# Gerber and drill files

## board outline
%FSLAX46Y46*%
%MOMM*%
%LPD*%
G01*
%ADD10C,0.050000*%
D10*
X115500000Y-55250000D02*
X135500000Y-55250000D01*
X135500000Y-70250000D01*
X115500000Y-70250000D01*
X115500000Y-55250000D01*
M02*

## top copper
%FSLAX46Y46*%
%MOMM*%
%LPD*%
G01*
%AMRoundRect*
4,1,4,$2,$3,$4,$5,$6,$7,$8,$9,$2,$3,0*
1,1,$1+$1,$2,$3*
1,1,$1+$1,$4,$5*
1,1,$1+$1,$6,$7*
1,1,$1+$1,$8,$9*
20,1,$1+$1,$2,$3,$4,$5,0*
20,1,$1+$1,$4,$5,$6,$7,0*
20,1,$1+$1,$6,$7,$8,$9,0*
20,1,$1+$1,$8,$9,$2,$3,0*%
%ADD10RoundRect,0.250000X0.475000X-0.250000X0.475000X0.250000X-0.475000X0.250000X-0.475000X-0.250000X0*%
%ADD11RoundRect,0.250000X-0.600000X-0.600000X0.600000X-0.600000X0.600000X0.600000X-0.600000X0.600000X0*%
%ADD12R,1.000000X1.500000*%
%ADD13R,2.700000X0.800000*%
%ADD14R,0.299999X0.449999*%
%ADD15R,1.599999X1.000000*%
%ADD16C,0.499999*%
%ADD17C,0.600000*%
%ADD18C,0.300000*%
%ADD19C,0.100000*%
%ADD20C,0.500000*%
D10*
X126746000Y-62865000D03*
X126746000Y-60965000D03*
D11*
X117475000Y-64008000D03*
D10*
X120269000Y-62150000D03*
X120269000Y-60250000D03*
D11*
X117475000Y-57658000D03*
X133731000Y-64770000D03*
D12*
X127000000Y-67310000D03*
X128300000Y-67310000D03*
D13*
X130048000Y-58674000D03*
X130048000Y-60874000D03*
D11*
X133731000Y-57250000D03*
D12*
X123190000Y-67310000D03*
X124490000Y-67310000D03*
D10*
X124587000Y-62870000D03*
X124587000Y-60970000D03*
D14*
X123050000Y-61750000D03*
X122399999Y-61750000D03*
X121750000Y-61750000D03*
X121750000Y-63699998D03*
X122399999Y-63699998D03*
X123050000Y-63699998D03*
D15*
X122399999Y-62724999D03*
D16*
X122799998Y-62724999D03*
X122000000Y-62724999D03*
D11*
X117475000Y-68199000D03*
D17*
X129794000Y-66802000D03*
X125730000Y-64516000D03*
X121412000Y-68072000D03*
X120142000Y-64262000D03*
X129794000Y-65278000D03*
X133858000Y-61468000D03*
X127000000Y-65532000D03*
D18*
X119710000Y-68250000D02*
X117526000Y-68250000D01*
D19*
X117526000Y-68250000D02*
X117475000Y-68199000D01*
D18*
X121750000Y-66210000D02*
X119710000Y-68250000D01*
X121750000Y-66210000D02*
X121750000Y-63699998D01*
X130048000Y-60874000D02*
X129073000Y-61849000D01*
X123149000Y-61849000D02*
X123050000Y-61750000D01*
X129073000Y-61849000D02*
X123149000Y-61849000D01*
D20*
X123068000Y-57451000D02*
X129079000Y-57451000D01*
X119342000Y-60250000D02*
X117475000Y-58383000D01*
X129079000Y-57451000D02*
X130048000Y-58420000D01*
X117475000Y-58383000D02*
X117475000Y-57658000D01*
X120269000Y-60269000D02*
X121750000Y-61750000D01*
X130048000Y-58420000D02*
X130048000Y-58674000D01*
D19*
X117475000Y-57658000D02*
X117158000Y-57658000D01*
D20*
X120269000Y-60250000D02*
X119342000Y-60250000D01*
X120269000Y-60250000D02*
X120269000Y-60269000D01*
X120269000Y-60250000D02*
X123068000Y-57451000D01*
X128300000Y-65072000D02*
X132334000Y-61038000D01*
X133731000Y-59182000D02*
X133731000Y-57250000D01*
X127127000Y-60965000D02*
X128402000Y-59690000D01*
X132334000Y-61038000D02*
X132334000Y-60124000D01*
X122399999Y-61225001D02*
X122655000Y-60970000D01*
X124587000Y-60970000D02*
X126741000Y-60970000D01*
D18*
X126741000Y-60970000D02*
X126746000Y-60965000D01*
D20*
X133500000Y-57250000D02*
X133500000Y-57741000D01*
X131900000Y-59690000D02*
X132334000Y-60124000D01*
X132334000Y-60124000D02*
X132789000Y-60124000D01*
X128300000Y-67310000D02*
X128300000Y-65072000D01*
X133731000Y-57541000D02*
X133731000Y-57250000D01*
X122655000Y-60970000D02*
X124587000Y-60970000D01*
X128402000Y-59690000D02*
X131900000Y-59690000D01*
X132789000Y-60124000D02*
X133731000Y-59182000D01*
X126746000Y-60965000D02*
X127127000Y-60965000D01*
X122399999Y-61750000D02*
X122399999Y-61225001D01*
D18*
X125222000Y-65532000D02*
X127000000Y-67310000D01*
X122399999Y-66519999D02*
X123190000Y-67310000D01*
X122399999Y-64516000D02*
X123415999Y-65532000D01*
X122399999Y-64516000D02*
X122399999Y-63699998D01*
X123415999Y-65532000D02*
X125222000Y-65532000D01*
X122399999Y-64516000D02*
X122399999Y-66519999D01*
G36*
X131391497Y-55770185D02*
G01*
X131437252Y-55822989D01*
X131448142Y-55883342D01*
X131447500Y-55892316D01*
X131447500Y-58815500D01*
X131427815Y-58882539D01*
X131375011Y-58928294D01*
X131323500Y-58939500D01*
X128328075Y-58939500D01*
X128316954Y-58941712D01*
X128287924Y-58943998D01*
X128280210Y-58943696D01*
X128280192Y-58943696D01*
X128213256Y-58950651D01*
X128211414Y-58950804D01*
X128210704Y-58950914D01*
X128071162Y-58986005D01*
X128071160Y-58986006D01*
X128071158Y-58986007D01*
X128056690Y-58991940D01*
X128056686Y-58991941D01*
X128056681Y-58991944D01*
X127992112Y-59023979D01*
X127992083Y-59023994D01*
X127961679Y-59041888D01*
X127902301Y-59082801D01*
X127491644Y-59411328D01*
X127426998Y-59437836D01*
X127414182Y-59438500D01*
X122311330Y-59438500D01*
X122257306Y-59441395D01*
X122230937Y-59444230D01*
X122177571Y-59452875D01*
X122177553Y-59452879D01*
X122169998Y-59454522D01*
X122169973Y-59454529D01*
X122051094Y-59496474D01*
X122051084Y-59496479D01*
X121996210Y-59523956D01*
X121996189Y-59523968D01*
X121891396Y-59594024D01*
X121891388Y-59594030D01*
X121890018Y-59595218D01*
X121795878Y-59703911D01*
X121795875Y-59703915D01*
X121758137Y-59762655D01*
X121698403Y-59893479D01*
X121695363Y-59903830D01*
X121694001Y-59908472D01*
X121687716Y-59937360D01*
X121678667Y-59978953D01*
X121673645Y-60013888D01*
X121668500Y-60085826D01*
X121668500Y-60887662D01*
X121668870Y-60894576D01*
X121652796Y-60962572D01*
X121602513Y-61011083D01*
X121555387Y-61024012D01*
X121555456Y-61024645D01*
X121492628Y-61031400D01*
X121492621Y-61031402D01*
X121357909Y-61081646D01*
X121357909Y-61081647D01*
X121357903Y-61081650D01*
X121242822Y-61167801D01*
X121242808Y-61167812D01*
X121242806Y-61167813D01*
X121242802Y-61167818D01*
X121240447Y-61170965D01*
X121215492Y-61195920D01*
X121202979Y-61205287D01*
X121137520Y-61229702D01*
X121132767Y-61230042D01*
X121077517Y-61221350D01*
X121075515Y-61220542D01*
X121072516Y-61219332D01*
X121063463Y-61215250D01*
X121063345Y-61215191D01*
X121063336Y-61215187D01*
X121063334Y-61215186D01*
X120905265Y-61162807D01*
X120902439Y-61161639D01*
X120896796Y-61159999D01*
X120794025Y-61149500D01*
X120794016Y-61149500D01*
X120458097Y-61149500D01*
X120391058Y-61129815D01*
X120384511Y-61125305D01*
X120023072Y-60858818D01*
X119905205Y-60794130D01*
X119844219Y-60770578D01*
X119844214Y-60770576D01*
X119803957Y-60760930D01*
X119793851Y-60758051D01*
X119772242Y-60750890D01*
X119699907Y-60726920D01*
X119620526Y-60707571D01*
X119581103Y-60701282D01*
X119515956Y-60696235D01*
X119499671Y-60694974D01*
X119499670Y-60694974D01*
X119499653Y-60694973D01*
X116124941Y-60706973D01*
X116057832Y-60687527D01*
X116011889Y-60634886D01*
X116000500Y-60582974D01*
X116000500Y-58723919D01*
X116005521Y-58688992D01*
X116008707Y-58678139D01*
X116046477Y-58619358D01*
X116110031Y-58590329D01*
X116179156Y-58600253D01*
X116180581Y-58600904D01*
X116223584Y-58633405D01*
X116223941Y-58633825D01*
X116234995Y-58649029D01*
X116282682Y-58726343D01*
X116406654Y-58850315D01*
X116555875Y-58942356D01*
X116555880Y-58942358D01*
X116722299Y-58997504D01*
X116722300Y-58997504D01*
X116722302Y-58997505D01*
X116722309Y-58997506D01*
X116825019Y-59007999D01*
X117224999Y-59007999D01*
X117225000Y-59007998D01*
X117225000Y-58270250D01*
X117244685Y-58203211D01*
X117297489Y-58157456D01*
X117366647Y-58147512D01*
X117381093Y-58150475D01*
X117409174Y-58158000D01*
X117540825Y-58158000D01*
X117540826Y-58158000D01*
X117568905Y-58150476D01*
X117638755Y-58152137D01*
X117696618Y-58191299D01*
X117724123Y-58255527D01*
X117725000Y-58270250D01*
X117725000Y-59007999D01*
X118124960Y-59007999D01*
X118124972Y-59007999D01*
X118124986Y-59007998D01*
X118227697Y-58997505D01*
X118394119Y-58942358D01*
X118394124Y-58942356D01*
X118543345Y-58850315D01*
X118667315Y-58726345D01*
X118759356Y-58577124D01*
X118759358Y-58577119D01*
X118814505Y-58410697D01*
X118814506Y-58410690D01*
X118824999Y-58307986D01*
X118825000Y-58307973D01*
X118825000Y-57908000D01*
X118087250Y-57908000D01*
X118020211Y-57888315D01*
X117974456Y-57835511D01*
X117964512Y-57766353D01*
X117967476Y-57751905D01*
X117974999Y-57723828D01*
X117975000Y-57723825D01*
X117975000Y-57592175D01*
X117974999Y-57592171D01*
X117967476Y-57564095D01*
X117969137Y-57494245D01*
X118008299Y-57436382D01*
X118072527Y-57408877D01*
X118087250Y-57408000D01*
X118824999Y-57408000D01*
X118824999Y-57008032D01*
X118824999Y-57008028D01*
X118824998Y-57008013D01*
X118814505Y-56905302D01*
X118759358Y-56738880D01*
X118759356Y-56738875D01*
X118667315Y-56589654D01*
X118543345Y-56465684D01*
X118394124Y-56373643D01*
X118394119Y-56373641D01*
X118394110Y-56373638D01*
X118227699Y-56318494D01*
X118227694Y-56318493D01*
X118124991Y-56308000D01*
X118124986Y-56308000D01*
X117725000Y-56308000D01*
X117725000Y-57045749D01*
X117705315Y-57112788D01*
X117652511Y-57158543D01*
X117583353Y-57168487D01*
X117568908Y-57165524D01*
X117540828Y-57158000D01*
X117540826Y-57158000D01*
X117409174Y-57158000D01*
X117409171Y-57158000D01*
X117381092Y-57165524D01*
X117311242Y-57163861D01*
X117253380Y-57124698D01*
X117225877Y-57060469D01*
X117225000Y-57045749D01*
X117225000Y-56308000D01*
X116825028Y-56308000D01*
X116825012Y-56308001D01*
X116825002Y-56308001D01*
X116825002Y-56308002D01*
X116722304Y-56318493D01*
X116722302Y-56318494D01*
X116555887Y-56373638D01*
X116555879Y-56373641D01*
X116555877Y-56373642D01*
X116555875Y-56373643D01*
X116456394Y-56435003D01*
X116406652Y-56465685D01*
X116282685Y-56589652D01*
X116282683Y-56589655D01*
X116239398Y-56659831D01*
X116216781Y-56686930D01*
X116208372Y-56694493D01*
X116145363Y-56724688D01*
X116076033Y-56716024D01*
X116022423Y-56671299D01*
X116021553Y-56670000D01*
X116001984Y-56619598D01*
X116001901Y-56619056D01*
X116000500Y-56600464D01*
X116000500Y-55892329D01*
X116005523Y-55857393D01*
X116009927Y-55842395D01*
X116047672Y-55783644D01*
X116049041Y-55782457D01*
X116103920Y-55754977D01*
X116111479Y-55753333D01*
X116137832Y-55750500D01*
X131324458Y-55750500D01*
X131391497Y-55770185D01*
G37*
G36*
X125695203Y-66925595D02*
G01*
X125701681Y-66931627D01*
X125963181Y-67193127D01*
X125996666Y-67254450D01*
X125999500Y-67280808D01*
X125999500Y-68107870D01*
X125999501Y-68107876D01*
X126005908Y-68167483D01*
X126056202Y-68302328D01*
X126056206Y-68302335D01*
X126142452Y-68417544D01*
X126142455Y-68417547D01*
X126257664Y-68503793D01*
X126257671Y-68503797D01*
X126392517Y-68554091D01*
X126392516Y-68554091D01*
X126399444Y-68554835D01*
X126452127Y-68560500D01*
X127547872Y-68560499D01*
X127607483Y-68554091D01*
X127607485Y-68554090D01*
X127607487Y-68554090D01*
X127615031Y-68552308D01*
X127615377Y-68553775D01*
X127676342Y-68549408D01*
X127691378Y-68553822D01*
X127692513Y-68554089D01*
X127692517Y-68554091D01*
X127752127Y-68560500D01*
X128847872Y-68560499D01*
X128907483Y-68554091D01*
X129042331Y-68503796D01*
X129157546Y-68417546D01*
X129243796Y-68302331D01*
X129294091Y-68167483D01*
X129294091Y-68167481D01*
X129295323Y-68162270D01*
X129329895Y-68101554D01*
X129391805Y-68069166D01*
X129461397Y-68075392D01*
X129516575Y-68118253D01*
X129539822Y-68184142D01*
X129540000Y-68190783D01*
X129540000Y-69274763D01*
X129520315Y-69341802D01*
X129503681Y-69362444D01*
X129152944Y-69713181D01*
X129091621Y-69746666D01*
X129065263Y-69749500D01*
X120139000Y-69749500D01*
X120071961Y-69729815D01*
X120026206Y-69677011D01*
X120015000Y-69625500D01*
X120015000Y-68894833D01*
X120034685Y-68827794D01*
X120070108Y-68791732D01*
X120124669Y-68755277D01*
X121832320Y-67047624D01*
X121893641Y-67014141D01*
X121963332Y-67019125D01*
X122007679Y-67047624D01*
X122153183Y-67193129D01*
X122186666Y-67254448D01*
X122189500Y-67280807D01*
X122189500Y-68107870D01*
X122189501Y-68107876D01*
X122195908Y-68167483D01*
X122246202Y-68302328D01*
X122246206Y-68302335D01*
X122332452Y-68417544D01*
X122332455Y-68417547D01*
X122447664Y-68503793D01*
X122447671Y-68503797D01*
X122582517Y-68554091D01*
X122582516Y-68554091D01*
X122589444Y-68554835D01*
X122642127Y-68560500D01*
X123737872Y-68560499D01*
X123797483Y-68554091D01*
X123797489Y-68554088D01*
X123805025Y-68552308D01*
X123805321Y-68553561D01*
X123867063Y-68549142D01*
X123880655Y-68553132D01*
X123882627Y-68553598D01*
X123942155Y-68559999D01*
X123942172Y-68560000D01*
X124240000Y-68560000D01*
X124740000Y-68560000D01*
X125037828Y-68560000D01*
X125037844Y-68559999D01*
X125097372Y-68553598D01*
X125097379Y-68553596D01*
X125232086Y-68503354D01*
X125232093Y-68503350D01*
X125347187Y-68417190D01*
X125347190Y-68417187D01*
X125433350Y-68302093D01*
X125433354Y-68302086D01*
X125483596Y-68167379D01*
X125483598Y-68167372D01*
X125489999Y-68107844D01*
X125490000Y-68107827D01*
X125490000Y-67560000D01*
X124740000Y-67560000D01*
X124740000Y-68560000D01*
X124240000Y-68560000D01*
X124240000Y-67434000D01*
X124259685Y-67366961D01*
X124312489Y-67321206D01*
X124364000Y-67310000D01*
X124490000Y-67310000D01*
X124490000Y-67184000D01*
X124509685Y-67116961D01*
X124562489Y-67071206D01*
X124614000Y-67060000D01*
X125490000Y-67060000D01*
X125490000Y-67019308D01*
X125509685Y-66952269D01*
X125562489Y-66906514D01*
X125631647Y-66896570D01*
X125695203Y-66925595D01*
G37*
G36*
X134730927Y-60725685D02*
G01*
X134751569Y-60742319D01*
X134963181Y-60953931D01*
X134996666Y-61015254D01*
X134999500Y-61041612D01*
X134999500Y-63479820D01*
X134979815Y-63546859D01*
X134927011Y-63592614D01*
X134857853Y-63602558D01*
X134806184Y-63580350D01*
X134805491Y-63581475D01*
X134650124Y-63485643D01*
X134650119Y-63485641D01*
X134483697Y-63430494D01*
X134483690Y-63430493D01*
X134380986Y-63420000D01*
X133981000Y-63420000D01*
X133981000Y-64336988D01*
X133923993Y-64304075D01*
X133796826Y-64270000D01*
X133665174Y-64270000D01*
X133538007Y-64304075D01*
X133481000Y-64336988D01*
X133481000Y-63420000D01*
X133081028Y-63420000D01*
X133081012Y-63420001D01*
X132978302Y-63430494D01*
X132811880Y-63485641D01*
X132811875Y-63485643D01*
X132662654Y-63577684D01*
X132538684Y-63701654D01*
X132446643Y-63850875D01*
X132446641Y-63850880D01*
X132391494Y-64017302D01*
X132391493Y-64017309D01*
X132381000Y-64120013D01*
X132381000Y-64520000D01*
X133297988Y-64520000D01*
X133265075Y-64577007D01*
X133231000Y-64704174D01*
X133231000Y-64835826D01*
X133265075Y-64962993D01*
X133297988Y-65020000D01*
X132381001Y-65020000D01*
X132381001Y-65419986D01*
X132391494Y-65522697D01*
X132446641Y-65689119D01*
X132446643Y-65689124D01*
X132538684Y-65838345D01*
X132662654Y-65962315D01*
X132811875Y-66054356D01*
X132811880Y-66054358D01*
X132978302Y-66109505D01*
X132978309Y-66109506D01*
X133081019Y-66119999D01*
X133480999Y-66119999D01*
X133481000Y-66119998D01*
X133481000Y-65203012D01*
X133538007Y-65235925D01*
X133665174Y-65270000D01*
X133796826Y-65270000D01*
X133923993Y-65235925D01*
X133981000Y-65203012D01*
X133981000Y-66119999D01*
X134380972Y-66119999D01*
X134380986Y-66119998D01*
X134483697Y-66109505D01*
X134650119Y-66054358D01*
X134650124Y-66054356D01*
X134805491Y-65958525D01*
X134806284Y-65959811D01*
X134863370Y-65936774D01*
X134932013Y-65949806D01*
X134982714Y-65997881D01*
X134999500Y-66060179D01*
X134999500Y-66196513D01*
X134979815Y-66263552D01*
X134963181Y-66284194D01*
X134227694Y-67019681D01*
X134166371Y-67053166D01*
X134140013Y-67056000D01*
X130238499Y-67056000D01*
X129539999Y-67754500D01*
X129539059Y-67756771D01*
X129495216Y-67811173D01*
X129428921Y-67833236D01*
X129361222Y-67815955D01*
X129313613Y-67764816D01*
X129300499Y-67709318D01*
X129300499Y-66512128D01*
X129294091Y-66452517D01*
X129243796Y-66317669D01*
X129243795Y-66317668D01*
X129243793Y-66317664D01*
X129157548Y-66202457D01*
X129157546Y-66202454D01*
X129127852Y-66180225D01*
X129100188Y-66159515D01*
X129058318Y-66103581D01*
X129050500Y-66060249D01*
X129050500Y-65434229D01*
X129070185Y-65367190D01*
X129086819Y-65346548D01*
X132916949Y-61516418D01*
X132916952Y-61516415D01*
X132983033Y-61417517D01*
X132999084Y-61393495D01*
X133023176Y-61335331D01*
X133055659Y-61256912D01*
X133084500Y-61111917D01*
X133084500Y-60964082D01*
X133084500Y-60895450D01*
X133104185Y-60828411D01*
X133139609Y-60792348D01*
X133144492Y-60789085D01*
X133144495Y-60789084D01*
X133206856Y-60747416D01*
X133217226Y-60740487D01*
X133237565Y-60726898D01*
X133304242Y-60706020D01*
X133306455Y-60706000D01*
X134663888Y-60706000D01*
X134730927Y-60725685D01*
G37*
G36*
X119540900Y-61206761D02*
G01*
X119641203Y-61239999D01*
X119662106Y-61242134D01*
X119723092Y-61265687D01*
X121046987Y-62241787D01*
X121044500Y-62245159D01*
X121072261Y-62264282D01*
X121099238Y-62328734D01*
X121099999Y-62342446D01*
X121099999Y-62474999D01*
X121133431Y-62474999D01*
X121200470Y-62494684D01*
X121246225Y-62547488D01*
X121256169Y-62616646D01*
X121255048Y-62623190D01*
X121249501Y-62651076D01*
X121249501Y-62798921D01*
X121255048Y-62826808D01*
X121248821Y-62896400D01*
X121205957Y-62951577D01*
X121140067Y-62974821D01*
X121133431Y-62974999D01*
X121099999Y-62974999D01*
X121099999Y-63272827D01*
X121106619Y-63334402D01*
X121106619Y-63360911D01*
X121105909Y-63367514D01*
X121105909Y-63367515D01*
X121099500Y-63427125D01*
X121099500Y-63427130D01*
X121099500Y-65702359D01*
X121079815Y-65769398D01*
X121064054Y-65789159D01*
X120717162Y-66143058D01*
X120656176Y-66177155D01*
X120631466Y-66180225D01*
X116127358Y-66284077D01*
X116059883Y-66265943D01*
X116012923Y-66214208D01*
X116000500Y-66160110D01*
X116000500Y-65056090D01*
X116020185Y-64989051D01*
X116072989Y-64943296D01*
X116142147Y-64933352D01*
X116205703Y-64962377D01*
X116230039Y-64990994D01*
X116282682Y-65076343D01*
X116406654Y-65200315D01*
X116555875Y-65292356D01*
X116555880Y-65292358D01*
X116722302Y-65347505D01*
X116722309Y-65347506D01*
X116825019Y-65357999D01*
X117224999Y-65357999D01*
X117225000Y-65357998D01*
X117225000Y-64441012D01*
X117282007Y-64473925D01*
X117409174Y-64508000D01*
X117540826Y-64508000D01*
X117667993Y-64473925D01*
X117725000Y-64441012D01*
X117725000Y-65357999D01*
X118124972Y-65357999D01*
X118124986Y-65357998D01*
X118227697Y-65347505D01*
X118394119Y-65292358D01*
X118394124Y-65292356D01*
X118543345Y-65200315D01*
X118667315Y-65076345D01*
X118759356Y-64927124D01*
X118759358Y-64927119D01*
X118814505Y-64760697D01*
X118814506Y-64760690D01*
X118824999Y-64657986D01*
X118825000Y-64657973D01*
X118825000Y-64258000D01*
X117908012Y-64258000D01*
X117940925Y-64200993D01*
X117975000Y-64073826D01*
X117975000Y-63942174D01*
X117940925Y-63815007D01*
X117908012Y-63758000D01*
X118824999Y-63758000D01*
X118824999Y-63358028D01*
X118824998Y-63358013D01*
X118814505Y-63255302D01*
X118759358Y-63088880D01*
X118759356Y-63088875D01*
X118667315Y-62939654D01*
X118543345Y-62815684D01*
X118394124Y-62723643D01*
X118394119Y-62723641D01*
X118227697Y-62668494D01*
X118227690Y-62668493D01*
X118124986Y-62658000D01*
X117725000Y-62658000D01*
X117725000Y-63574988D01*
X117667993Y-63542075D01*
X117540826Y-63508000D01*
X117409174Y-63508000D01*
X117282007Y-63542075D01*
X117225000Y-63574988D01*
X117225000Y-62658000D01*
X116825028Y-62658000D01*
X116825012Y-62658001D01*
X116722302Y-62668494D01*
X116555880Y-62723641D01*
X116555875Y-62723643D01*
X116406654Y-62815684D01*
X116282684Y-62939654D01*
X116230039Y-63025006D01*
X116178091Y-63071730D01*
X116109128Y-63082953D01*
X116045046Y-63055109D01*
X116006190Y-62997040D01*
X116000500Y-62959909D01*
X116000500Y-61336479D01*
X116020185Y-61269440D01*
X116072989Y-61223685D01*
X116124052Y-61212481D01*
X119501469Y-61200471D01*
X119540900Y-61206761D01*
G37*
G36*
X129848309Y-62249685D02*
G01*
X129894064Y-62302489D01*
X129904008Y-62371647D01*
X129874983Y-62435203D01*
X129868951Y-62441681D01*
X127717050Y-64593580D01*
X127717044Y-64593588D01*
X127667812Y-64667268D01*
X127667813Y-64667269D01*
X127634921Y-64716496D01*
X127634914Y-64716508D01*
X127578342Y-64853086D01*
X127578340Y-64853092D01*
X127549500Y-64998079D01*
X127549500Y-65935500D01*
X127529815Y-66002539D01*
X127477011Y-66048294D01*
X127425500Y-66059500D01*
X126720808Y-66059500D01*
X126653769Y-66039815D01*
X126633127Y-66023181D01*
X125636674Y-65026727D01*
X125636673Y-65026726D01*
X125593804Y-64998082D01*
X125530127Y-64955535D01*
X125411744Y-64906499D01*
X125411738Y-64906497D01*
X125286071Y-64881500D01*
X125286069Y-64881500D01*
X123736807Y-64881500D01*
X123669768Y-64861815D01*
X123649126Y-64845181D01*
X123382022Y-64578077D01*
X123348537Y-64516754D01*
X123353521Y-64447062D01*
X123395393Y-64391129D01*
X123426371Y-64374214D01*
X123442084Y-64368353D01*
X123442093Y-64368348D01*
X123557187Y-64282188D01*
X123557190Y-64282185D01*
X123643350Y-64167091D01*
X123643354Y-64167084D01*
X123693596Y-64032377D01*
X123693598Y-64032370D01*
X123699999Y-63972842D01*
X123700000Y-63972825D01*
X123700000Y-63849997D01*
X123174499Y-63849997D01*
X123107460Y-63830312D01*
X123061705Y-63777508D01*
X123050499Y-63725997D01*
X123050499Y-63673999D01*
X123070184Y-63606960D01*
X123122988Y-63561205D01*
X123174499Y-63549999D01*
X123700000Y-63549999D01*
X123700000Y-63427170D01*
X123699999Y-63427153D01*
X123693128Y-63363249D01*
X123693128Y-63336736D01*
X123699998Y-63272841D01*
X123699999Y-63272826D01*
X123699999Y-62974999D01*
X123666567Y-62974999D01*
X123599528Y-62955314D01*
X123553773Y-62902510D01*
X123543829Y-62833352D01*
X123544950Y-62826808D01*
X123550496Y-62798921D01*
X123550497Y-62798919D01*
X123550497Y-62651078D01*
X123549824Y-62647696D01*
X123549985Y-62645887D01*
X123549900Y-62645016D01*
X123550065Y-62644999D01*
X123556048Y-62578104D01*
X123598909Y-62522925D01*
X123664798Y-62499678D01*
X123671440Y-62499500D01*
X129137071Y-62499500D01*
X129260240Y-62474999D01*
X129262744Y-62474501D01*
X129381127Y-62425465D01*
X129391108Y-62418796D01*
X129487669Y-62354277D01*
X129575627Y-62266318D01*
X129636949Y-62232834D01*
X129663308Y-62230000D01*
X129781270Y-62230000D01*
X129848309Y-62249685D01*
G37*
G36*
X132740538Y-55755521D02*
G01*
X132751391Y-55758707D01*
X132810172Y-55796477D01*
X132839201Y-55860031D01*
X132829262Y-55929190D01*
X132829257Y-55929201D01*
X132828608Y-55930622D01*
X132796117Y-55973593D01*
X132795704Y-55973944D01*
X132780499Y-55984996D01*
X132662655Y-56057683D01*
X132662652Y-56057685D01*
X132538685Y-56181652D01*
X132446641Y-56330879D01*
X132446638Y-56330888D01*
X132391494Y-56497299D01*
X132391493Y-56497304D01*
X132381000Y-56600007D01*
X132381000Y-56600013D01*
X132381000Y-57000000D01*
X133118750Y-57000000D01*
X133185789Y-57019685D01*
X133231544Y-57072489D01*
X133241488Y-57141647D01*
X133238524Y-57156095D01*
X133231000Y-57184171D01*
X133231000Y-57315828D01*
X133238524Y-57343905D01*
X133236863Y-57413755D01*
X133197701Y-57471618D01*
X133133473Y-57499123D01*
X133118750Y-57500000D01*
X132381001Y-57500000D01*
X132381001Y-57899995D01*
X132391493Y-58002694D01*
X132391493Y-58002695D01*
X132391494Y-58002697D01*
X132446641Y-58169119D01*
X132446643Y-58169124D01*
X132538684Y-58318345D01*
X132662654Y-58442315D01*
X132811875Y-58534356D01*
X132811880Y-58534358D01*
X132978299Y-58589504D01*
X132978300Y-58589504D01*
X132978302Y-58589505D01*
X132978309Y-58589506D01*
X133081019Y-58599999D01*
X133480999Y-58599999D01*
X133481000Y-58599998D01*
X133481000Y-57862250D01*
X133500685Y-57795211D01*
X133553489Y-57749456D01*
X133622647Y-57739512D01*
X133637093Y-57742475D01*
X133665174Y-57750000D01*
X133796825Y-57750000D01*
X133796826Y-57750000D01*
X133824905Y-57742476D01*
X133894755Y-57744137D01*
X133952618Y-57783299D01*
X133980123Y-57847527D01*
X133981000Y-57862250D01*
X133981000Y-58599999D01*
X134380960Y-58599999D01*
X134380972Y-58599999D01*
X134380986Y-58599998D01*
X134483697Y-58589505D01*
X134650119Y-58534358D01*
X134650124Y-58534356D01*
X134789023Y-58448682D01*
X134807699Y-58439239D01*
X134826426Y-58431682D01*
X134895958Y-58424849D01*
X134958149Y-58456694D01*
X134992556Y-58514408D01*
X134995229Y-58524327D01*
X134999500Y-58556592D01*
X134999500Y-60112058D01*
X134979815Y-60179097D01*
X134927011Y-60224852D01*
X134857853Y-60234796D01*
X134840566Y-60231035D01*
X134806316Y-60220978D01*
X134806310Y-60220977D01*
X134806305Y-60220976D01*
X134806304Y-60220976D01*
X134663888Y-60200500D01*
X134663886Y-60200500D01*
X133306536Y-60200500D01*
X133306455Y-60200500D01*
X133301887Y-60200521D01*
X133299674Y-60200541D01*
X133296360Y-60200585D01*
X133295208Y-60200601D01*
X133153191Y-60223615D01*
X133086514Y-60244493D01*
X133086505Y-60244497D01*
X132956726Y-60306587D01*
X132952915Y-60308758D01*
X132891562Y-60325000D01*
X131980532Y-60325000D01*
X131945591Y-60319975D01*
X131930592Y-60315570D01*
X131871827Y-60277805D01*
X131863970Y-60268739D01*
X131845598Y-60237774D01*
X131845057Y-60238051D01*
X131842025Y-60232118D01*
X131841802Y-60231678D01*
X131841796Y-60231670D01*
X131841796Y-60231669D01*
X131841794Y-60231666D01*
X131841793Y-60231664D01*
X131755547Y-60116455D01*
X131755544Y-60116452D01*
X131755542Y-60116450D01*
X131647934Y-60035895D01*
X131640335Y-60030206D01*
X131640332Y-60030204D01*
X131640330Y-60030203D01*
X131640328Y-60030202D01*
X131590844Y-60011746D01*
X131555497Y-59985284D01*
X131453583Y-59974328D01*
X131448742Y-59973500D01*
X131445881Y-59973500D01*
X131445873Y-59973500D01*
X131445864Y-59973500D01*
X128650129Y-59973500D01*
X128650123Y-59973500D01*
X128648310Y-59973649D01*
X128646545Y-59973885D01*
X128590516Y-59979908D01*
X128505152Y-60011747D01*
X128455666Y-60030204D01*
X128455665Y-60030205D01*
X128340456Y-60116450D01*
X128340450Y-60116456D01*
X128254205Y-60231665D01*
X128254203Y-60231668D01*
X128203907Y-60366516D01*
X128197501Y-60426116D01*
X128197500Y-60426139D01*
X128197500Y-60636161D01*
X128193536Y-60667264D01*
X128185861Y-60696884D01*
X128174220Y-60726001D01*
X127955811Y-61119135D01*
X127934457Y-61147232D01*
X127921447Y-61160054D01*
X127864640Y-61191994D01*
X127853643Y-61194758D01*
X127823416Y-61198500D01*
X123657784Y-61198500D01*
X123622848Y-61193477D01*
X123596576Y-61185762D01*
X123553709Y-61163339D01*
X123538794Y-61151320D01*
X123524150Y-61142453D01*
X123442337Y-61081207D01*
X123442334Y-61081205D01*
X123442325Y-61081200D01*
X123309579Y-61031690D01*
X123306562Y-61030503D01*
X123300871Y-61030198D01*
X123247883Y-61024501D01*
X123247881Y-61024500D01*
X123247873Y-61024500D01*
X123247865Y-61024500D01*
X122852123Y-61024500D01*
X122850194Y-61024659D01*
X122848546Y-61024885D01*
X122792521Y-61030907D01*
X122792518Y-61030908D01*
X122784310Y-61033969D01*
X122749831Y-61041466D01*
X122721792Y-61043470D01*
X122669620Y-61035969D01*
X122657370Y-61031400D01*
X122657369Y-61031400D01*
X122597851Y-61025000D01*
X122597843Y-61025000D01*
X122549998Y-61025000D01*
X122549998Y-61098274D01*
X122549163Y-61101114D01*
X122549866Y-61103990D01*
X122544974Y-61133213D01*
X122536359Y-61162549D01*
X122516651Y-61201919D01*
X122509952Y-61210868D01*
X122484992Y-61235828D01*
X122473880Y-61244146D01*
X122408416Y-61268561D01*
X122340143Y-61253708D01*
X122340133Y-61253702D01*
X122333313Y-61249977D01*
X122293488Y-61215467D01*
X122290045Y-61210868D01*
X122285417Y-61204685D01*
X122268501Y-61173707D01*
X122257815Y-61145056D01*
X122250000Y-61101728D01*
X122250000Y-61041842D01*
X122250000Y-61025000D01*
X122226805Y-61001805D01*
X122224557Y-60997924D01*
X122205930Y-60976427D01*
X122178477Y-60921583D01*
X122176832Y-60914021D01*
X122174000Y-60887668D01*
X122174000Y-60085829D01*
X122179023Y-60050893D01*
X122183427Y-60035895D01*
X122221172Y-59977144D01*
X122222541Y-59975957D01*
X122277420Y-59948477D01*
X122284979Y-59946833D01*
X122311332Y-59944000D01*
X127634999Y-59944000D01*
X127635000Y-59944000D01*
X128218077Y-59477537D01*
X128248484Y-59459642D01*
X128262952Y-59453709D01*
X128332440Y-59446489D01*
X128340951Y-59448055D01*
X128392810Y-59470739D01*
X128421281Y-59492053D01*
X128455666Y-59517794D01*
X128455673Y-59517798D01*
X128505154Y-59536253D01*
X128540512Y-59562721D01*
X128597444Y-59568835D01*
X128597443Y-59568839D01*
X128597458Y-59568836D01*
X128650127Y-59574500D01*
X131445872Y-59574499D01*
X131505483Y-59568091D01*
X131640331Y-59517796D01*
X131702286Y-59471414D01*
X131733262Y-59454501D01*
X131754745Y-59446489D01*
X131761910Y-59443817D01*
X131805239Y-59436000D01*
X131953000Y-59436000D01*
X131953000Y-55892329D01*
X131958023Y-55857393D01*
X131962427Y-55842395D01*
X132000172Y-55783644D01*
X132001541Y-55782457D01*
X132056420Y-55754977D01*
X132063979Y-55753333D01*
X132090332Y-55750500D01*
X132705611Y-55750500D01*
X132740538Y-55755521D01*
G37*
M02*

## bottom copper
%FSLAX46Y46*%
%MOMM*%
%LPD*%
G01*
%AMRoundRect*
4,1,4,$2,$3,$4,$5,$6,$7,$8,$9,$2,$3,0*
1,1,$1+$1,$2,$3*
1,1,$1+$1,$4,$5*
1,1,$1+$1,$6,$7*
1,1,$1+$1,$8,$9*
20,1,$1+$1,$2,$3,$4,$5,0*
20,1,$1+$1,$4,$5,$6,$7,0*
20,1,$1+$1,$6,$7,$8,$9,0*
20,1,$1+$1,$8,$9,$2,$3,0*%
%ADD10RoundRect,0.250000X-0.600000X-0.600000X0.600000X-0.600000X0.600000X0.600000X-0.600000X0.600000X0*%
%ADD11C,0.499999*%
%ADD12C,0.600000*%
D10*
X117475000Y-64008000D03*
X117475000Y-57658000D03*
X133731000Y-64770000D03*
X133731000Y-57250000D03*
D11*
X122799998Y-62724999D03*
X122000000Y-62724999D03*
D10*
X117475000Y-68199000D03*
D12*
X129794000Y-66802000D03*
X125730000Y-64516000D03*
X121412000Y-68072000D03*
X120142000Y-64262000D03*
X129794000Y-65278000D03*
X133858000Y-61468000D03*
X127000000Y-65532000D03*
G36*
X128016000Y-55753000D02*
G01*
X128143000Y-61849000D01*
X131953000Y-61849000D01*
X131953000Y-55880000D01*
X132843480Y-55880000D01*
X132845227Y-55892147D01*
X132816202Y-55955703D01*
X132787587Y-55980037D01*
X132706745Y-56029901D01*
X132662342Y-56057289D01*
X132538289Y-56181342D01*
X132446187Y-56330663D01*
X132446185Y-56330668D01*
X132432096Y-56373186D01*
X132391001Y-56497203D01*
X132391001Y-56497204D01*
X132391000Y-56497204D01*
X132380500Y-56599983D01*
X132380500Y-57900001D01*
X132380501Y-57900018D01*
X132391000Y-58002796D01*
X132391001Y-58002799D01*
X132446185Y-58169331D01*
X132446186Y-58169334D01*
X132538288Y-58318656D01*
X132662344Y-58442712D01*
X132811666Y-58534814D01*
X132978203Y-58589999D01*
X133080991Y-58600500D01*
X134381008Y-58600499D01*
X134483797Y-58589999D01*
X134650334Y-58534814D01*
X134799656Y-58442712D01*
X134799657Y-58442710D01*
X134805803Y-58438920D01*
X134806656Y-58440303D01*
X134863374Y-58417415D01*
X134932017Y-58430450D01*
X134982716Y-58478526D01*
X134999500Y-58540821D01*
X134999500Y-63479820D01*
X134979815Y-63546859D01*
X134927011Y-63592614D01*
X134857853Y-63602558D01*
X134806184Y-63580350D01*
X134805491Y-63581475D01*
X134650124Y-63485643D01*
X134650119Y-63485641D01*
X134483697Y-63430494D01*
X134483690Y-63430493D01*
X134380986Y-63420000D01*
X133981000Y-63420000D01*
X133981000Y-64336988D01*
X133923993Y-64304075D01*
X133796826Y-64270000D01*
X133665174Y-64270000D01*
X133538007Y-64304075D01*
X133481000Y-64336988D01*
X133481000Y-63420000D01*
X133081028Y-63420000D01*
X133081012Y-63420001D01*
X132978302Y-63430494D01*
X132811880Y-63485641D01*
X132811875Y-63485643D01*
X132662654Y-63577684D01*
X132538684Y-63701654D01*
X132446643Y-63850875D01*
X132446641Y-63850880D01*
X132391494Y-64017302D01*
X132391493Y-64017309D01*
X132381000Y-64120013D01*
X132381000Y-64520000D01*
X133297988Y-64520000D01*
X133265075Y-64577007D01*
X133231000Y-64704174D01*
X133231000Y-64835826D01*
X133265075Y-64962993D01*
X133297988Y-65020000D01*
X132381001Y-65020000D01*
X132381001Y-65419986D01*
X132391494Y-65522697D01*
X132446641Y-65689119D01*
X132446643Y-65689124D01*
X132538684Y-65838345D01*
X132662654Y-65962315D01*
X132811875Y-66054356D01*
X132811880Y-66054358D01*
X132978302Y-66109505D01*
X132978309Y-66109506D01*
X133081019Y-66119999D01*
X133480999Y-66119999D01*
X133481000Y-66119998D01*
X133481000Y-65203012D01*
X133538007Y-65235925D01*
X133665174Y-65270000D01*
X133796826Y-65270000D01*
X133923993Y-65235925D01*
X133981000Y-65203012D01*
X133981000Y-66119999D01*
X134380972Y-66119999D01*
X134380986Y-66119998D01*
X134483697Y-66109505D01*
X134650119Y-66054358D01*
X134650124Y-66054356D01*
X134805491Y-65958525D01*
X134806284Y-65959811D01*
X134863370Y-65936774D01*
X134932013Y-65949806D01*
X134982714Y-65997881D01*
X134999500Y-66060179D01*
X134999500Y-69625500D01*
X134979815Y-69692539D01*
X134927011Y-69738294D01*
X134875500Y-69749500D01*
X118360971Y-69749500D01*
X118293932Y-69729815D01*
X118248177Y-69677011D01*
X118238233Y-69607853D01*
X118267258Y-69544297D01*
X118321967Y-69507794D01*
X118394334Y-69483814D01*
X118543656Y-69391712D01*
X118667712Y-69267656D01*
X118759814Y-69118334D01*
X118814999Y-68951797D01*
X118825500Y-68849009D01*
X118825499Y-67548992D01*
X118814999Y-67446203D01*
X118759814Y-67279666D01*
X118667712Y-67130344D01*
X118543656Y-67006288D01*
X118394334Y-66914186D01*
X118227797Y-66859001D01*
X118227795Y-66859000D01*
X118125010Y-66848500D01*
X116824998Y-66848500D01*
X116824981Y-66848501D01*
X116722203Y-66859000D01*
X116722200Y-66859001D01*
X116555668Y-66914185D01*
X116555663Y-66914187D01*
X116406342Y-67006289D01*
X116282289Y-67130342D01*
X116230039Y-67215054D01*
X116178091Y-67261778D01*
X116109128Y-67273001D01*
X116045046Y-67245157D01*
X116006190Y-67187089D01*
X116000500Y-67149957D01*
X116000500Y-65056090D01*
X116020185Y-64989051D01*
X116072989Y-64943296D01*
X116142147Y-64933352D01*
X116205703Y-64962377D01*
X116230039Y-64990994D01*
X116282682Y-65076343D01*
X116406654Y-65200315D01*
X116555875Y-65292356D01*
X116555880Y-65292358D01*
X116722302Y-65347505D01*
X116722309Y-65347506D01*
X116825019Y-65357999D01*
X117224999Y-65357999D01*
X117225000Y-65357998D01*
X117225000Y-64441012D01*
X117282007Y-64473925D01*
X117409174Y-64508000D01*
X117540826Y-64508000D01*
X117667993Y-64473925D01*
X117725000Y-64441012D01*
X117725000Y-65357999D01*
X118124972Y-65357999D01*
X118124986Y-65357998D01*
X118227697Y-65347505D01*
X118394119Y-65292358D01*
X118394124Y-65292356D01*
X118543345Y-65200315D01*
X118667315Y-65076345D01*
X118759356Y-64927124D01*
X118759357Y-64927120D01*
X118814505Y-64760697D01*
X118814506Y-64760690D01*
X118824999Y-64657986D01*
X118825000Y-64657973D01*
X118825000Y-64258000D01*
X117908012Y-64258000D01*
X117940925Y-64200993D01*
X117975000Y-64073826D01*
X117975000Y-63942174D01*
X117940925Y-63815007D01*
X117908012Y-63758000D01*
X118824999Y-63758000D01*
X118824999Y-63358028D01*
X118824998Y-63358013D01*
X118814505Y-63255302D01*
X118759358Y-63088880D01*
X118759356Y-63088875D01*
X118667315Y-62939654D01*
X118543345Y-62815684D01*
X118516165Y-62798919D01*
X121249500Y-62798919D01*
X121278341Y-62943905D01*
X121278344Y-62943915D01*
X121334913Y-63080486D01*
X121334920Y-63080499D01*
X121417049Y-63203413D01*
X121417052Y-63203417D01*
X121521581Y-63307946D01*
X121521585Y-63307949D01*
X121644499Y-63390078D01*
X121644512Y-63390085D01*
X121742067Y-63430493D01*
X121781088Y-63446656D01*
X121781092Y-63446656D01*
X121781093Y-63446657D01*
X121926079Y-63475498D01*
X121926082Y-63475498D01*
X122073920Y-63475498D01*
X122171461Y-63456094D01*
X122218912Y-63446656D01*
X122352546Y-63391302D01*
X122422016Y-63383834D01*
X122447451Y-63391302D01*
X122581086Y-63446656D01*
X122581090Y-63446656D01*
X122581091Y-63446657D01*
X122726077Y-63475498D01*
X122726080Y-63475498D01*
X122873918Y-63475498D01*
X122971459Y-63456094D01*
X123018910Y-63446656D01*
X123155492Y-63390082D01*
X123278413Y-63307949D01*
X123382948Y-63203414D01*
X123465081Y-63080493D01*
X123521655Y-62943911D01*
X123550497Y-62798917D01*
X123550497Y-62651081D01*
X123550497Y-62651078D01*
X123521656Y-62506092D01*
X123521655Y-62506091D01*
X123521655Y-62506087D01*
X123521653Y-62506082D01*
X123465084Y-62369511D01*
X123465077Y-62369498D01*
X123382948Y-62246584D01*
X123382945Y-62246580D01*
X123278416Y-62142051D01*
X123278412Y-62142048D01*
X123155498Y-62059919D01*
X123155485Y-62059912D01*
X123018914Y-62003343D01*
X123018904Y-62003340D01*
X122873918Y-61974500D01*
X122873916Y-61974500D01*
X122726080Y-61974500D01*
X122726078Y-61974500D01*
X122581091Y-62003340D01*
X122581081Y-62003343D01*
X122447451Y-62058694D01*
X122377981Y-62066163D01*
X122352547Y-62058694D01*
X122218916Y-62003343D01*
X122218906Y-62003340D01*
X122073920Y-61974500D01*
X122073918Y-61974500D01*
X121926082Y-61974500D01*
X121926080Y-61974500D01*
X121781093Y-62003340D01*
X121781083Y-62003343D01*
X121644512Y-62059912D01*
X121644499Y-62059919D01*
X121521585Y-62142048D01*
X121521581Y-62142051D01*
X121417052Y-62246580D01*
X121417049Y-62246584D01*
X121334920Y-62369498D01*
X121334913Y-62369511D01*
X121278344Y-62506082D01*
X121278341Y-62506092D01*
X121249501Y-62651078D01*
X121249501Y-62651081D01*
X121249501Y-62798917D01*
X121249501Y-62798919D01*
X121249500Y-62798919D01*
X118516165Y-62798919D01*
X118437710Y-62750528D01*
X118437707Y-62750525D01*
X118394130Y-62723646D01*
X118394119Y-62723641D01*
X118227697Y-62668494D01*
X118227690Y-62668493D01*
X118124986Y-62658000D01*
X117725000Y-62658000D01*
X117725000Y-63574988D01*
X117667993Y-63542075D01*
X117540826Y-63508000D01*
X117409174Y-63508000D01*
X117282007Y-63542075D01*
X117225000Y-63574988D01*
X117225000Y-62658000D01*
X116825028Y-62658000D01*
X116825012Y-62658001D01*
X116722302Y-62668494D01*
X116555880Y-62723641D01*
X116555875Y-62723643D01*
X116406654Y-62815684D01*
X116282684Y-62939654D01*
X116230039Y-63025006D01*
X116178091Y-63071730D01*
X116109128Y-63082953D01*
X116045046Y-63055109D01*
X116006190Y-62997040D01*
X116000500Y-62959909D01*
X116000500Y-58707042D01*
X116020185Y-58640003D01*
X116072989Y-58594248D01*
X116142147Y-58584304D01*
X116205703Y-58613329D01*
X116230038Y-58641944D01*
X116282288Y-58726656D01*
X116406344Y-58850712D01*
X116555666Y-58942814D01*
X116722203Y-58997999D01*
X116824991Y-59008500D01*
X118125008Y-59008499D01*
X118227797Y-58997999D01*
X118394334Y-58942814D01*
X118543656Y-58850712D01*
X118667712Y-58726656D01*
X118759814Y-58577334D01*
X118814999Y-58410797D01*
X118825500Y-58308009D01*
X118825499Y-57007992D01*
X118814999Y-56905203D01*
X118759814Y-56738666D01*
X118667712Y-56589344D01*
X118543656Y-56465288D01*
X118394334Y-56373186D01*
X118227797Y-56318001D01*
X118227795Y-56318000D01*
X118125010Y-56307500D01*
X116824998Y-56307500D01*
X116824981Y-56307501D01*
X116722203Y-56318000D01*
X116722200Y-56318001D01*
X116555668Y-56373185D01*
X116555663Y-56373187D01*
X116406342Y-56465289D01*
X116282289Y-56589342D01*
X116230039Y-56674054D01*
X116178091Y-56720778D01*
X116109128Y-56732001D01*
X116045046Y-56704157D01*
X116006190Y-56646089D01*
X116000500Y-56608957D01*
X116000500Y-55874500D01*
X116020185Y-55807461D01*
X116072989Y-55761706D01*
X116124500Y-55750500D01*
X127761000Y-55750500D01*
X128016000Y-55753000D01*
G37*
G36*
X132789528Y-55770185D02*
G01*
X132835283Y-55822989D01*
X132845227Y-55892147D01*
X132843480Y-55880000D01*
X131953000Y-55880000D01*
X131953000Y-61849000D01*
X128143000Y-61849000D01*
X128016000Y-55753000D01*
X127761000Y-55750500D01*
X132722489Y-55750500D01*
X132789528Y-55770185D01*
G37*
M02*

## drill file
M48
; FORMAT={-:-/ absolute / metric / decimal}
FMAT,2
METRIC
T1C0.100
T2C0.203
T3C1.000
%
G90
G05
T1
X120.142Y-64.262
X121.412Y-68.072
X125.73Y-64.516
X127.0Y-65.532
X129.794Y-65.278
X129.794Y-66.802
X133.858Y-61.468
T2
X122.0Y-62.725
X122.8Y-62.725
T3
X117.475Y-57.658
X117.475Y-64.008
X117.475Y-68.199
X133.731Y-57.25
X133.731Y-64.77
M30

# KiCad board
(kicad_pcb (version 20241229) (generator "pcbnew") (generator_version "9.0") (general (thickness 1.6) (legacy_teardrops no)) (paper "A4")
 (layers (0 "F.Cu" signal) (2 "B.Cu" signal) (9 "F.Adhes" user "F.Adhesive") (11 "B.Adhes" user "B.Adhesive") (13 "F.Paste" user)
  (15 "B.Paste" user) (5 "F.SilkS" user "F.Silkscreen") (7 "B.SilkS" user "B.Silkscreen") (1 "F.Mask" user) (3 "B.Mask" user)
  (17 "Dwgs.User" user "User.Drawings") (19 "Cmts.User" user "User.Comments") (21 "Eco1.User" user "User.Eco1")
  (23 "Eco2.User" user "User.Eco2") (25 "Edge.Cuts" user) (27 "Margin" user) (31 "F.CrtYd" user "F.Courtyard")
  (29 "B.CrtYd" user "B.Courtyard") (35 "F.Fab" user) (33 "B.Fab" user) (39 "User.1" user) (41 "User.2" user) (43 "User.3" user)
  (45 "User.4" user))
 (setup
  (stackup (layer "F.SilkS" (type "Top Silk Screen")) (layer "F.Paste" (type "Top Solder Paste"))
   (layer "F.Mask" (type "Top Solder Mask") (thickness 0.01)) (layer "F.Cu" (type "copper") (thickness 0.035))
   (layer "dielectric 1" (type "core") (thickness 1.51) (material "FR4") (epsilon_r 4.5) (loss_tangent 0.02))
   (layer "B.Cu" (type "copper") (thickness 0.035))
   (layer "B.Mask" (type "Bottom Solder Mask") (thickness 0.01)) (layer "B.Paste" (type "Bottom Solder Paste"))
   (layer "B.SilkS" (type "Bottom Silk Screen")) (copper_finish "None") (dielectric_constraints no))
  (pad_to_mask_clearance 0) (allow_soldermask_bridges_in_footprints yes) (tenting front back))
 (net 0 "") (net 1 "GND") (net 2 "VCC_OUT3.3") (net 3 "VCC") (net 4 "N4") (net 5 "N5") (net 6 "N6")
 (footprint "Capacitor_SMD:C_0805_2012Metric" (layer "F.Cu") (at 126.746 61.915 90)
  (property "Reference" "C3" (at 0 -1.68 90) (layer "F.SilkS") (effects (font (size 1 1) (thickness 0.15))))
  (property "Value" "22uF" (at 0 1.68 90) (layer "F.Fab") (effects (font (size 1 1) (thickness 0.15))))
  (pad "1" smd roundrect (at -0.95 0 90) (size 1 1.45) (layers "F.Cu" "F.Mask" "F.Paste") (roundrect_rratio 0.25) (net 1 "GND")
   (zone_connect 2))
  (pad "2" smd roundrect (at 0.95 0 90) (size 1 1.45) (layers "F.Cu" "F.Mask" "F.Paste") (roundrect_rratio 0.25) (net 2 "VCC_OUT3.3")
   (zone_connect 2)))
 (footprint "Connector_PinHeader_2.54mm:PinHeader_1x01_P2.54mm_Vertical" (layer "F.Cu") (at 117.475 64.008)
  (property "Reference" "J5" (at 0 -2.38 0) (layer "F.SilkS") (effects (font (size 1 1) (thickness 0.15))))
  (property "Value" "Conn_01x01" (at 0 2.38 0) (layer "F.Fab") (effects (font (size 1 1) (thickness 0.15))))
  (pad "1" thru_hole roundrect (at 0 0) (size 1.7 1.7) (drill 1) (layers "*.Cu" "*.Mask") (remove_unused_layers no)
   (roundrect_rratio 0.1470588235) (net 1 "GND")))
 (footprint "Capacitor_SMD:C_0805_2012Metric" (layer "F.Cu") (at 120.269 61.2 90)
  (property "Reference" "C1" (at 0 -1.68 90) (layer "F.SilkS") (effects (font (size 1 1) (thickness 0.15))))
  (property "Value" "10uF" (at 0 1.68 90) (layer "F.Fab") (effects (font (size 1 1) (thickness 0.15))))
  (pad "1" smd roundrect (at -0.95 0 90) (size 1 1.45) (layers "F.Cu" "F.Mask" "F.Paste") (roundrect_rratio 0.25) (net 1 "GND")
   (zone_connect 2))
  (pad "2" smd roundrect (at 0.95 0 90) (size 1 1.45) (layers "F.Cu" "F.Mask" "F.Paste") (roundrect_rratio 0.25) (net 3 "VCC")
   (zone_connect 2) (thermal_gap 1)))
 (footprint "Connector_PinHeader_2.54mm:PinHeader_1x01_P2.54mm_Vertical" (layer "F.Cu") (at 117.475 57.658)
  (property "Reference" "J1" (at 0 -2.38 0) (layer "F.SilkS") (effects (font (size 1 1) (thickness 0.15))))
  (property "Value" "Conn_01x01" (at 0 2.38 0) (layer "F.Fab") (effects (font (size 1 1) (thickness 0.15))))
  (pad "1" thru_hole roundrect (at 0 0) (size 1.7 1.7) (drill 1) (layers "*.Cu" "*.Mask") (remove_unused_layers no)
   (roundrect_rratio 0.1470588235) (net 3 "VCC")))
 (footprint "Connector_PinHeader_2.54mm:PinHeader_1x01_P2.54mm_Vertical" (layer "F.Cu") (at 133.731 64.77)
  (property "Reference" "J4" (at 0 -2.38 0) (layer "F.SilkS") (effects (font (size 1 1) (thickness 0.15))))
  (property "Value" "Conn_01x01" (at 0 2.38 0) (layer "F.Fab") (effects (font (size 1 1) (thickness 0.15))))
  (pad "1" thru_hole roundrect (at 0 0) (size 1.7 1.7) (drill 1) (layers "*.Cu" "*.Mask") (remove_unused_layers no)
   (roundrect_rratio 0.1470588235) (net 1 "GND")))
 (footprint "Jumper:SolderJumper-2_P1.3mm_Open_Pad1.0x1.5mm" (layer "F.Cu") (at 127.65 67.31)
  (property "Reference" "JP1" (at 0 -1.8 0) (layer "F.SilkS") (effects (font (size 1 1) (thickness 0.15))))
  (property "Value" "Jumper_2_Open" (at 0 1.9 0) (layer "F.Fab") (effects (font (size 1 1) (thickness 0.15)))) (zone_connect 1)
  (pad "1" smd rect (at -0.65 0) (size 1 1.5) (layers "F.Cu" "F.Mask") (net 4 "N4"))
  (pad "2" smd rect (at 0.65 0) (size 1 1.5) (layers "F.Cu" "F.Mask") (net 2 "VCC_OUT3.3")))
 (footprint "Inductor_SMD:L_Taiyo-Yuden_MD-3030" (layer "F.Cu") (at 130.048 59.774 -90)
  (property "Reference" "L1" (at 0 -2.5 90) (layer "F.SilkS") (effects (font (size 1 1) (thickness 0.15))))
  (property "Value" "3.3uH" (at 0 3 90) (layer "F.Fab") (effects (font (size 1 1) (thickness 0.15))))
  (pad "1" smd rect (at -1.1 0 270) (size 0.8 2.7) (layers "F.Cu" "F.Mask" "F.Paste") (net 3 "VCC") (zone_connect 2))
  (pad "2" smd rect (at 1.1 0 270) (size 0.8 2.7) (layers "F.Cu" "F.Mask" "F.Paste") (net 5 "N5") (zone_connect 2)))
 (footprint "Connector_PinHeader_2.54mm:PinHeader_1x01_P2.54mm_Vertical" (layer "F.Cu") (at 133.731 57.25)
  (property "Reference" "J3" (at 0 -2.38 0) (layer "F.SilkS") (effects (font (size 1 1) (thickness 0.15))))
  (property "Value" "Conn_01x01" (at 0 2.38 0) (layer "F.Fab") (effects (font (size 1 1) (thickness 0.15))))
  (pad "1" thru_hole roundrect (at 0 0) (size 1.7 1.7) (drill 1) (layers "*.Cu" "*.Mask") (remove_unused_layers no)
   (roundrect_rratio 0.1470588235) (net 2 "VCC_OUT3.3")))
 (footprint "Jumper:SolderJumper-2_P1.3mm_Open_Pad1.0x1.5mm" (layer "F.Cu") (at 123.84 67.31)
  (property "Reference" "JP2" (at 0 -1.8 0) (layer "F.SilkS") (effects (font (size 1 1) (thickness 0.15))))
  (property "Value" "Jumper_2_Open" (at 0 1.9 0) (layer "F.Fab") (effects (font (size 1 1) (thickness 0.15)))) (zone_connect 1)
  (pad "1" smd rect (at -0.65 0) (size 1 1.5) (layers "F.Cu" "F.Mask") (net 4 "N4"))
  (pad "2" smd rect (at 0.65 0) (size 1 1.5) (layers "F.Cu" "F.Mask") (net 1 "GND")))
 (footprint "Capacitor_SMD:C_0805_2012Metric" (layer "F.Cu") (at 124.587 61.92 90)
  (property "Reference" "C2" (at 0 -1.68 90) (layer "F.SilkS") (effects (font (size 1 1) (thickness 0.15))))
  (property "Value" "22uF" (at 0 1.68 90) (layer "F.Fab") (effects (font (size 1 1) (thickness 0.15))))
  (pad "1" smd roundrect (at -0.95 0 90) (size 1 1.45) (layers "F.Cu" "F.Mask" "F.Paste") (roundrect_rratio 0.25) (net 1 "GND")
   (zone_connect 2))
  (pad "2" smd roundrect (at 0.95 0 90) (size 1 1.45) (layers "F.Cu" "F.Mask" "F.Paste") (roundrect_rratio 0.25) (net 2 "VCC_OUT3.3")
   (zone_connect 2)))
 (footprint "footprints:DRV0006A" (layer "F.Cu") (at 122.399999 62.724999 -90)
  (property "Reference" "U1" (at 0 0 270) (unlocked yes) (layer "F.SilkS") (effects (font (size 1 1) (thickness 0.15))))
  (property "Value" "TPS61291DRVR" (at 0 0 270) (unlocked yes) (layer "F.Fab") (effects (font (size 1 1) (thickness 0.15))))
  (pad "1" smd rect (at -0.974999 -0.650001) (size 0.299999 0.449999) (layers "F.Cu" "F.Mask" "F.Paste") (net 5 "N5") (solder_mask_margin 0))
  (pad "2" smd rect (at -0.974999 0) (size 0.299999 0.449999) (layers "F.Cu" "F.Mask" "F.Paste") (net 2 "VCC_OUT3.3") (solder_mask_margin 0))
  (pad "3" smd rect (at -0.974999 0.649999) (size 0.299999 0.449999) (layers "F.Cu" "F.Mask" "F.Paste") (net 3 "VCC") (solder_mask_margin 0))
  (pad "4" smd rect (at 0.974999 0.649999) (size 0.299999 0.449999) (layers "F.Cu" "F.Mask" "F.Paste") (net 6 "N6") (solder_mask_margin 0))
  (pad "5" smd rect (at 0.974999 0) (size 0.299999 0.449999) (layers "F.Cu" "F.Mask" "F.Paste") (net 4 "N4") (solder_mask_margin 0)
   (clearance 0))
  (pad "6" smd rect (at 0.974999 -0.650001) (size 0.299999 0.449999) (layers "F.Cu" "F.Mask" "F.Paste") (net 1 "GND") (solder_mask_margin 0))
  (pad "7" smd rect (at 0 0 270) (size 1 1.599999) (layers "F.Cu" "F.Mask" "F.Paste") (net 1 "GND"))
  (pad "V" thru_hole circle (at 0 -0.399999 270) (size 0.499999 0.499999) (drill 0.2032) (layers "*.Cu" "*.Mask") (remove_unused_layers no))
  (pad "V" thru_hole circle (at 0 0.399999 270) (size 0.499999 0.499999) (drill 0.2032) (layers "*.Cu" "*.Mask") (remove_unused_layers no)))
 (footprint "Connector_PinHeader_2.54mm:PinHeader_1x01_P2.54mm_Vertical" (layer "F.Cu") (at 117.475 68.199)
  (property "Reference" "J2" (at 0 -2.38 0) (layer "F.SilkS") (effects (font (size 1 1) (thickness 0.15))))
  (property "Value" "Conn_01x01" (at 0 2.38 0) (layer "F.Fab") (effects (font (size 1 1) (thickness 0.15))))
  (pad "1" thru_hole roundrect (at 0 0) (size 1.7 1.7) (drill 1) (layers "*.Cu" "*.Mask") (remove_unused_layers no)
   (roundrect_rratio 0.1470588235) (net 6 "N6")))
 (gr_rect (start 115.5 55.25) (end 135.5 70.25) (stroke (width 0.05) (type default)) (fill no) (layer "Edge.Cuts"))
 (via (at 129.794 66.802) (size 0.6) (drill 0.1) (layers "F.Cu" "B.Cu") (free yes) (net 1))
 (via (at 125.73 64.516) (size 0.6) (drill 0.1) (layers "F.Cu" "B.Cu") (free yes) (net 1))
 (via (at 121.412 68.072) (size 0.6) (drill 0.1) (layers "F.Cu" "B.Cu") (free yes) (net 1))
 (via (at 120.142 64.262) (size 0.6) (drill 0.1) (layers "F.Cu" "B.Cu") (free yes) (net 1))
 (via (at 129.794 65.278) (size 0.6) (drill 0.1) (layers "F.Cu" "B.Cu") (free yes) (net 1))
 (via (at 133.858 61.468) (size 0.6) (drill 0.1) (layers "F.Cu" "B.Cu") (free yes) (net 1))
 (via (at 127 65.532) (size 0.6) (drill 0.1) (layers "F.Cu" "B.Cu") (free yes) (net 1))
 (segment (start 119.71 68.25) (end 117.526 68.25) (width 0.3) (layer "F.Cu") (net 6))
 (segment (start 117.526 68.25) (end 117.475 68.199) (width 0.1) (layer "F.Cu") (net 6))
 (segment (start 121.75 66.21) (end 119.71 68.25) (width 0.3) (layer "F.Cu") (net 6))
 (segment (start 121.75 66.21) (end 121.75 63.699998) (width 0.3) (layer "F.Cu") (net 6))
 (segment (start 130.048 60.874) (end 129.073 61.849) (width 0.3) (layer "F.Cu") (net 5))
 (segment (start 123.149 61.849) (end 123.05 61.75) (width 0.3) (layer "F.Cu") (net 5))
 (segment (start 129.073 61.849) (end 123.149 61.849) (width 0.3) (layer "F.Cu") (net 5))
 (segment (start 123.068 57.451) (end 129.079 57.451) (width 0.5) (layer "F.Cu") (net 3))
 (segment (start 119.342 60.25) (end 117.475 58.383) (width 0.5) (layer "F.Cu") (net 3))
 (segment (start 129.079 57.451) (end 130.048 58.42) (width 0.5) (layer "F.Cu") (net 3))
 (segment (start 117.475 58.383) (end 117.475 57.658) (width 0.5) (layer "F.Cu") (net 3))
 (segment (start 120.269 60.269) (end 121.75 61.75) (width 0.5) (layer "F.Cu") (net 3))
 (segment (start 130.048 58.42) (end 130.048 58.674) (width 0.5) (layer "F.Cu") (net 3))
 (segment (start 117.475 57.658) (end 117.158 57.658) (width 0.1) (layer "F.Cu") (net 3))
 (segment (start 120.269 60.25) (end 119.342 60.25) (width 0.5) (layer "F.Cu") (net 3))
 (segment (start 120.269 60.25) (end 120.269 60.269) (width 0.5) (layer "F.Cu") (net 3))
 (segment (start 120.269 60.25) (end 123.068 57.451) (width 0.5) (layer "F.Cu") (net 3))
 (segment (start 128.3 65.072) (end 132.334 61.038) (width 0.5) (layer "F.Cu") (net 2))
 (segment (start 133.731 59.182) (end 133.731 57.25) (width 0.5) (layer "F.Cu") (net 2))
 (segment (start 127.127 60.965) (end 128.402 59.69) (width 0.5) (layer "F.Cu") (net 2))
 (segment (start 132.334 61.038) (end 132.334 60.124) (width 0.5) (layer "F.Cu") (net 2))
 (segment (start 122.399999 61.225001) (end 122.655 60.97) (width 0.5) (layer "F.Cu") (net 2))
 (segment (start 124.587 60.97) (end 126.741 60.97) (width 0.5) (layer "F.Cu") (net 2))
 (segment (start 126.741 60.97) (end 126.746 60.965) (width 0.3) (layer "F.Cu") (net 2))
 (segment (start 133.5 57.25) (end 133.5 57.741) (width 0.5) (layer "F.Cu") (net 2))
 (segment (start 131.9 59.69) (end 132.334 60.124) (width 0.5) (layer "F.Cu") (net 2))
 (segment (start 132.334 60.124) (end 132.789 60.124) (width 0.5) (layer "F.Cu") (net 2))
 (segment (start 128.3 67.31) (end 128.3 65.072) (width 0.5) (layer "F.Cu") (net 2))
 (segment (start 133.731 57.541) (end 133.731 57.25) (width 0.5) (layer "F.Cu") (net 2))
 (segment (start 122.655 60.97) (end 124.587 60.97) (width 0.5) (layer "F.Cu") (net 2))
 (segment (start 128.402 59.69) (end 131.9 59.69) (width 0.5) (layer "F.Cu") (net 2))
 (segment (start 132.789 60.124) (end 133.731 59.182) (width 0.5) (layer "F.Cu") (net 2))
 (segment (start 126.746 60.965) (end 127.127 60.965) (width 0.5) (layer "F.Cu") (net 2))
 (segment (start 122.399999 61.75) (end 122.399999 61.225001) (width 0.5) (layer "F.Cu") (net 2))
 (segment (start 125.222 65.532) (end 127 67.31) (width 0.3) (layer "F.Cu") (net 4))
 (segment (start 122.399999 66.519999) (end 123.19 67.31) (width 0.3) (layer "F.Cu") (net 4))
 (segment (start 122.399999 64.516) (end 123.415999 65.532) (width 0.3) (layer "F.Cu") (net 4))
 (segment (start 122.399999 64.516) (end 122.399999 63.699998) (width 0.3) (layer "F.Cu") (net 4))
 (segment (start 123.415999 65.532) (end 125.222 65.532) (width 0.3) (layer "F.Cu") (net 4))
 (segment (start 122.399999 64.516) (end 122.399999 66.519999) (width 0.3) (layer "F.Cu") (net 4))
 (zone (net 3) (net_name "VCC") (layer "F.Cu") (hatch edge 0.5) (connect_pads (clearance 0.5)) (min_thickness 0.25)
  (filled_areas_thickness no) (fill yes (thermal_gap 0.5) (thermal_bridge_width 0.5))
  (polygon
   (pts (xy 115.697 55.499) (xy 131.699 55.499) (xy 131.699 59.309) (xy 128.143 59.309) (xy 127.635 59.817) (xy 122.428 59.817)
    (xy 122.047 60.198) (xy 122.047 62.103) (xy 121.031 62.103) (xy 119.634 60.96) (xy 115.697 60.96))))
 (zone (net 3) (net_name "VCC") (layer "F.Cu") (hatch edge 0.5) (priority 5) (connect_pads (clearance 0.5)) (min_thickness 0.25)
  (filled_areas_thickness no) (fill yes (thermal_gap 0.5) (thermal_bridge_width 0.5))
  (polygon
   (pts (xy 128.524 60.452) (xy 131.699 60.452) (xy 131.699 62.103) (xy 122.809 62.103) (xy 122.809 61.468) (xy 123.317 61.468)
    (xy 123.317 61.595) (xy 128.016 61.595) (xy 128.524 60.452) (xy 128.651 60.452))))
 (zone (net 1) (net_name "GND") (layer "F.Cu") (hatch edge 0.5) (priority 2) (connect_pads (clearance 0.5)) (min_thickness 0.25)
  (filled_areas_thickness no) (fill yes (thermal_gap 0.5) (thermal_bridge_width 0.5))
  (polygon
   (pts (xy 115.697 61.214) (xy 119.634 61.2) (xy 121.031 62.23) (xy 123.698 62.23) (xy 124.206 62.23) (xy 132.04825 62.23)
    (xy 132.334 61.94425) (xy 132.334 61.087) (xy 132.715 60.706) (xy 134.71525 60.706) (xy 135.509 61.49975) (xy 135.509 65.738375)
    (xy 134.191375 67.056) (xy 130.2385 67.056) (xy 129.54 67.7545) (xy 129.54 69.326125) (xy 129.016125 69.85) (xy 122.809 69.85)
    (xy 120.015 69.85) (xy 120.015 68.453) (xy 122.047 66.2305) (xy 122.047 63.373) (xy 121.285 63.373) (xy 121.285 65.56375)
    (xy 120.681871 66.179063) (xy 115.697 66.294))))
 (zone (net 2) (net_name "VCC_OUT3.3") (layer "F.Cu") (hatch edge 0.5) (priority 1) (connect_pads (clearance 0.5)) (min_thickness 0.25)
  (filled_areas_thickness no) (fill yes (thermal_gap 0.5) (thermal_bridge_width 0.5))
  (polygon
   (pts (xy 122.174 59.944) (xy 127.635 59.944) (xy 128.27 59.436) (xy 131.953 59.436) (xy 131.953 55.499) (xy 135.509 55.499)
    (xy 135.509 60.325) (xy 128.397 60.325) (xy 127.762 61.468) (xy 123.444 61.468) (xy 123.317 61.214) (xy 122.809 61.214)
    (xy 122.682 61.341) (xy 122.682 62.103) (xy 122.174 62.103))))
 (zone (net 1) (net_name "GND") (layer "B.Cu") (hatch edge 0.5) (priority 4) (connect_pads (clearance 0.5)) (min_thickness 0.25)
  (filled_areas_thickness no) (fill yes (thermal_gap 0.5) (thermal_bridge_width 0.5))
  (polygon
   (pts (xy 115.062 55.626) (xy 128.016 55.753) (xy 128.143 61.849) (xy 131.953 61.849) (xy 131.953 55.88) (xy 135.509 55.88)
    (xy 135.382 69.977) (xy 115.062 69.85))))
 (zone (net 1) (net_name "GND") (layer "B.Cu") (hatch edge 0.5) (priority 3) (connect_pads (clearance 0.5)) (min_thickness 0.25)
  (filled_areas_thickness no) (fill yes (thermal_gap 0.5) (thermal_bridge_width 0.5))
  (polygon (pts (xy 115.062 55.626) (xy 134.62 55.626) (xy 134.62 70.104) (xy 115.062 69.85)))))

